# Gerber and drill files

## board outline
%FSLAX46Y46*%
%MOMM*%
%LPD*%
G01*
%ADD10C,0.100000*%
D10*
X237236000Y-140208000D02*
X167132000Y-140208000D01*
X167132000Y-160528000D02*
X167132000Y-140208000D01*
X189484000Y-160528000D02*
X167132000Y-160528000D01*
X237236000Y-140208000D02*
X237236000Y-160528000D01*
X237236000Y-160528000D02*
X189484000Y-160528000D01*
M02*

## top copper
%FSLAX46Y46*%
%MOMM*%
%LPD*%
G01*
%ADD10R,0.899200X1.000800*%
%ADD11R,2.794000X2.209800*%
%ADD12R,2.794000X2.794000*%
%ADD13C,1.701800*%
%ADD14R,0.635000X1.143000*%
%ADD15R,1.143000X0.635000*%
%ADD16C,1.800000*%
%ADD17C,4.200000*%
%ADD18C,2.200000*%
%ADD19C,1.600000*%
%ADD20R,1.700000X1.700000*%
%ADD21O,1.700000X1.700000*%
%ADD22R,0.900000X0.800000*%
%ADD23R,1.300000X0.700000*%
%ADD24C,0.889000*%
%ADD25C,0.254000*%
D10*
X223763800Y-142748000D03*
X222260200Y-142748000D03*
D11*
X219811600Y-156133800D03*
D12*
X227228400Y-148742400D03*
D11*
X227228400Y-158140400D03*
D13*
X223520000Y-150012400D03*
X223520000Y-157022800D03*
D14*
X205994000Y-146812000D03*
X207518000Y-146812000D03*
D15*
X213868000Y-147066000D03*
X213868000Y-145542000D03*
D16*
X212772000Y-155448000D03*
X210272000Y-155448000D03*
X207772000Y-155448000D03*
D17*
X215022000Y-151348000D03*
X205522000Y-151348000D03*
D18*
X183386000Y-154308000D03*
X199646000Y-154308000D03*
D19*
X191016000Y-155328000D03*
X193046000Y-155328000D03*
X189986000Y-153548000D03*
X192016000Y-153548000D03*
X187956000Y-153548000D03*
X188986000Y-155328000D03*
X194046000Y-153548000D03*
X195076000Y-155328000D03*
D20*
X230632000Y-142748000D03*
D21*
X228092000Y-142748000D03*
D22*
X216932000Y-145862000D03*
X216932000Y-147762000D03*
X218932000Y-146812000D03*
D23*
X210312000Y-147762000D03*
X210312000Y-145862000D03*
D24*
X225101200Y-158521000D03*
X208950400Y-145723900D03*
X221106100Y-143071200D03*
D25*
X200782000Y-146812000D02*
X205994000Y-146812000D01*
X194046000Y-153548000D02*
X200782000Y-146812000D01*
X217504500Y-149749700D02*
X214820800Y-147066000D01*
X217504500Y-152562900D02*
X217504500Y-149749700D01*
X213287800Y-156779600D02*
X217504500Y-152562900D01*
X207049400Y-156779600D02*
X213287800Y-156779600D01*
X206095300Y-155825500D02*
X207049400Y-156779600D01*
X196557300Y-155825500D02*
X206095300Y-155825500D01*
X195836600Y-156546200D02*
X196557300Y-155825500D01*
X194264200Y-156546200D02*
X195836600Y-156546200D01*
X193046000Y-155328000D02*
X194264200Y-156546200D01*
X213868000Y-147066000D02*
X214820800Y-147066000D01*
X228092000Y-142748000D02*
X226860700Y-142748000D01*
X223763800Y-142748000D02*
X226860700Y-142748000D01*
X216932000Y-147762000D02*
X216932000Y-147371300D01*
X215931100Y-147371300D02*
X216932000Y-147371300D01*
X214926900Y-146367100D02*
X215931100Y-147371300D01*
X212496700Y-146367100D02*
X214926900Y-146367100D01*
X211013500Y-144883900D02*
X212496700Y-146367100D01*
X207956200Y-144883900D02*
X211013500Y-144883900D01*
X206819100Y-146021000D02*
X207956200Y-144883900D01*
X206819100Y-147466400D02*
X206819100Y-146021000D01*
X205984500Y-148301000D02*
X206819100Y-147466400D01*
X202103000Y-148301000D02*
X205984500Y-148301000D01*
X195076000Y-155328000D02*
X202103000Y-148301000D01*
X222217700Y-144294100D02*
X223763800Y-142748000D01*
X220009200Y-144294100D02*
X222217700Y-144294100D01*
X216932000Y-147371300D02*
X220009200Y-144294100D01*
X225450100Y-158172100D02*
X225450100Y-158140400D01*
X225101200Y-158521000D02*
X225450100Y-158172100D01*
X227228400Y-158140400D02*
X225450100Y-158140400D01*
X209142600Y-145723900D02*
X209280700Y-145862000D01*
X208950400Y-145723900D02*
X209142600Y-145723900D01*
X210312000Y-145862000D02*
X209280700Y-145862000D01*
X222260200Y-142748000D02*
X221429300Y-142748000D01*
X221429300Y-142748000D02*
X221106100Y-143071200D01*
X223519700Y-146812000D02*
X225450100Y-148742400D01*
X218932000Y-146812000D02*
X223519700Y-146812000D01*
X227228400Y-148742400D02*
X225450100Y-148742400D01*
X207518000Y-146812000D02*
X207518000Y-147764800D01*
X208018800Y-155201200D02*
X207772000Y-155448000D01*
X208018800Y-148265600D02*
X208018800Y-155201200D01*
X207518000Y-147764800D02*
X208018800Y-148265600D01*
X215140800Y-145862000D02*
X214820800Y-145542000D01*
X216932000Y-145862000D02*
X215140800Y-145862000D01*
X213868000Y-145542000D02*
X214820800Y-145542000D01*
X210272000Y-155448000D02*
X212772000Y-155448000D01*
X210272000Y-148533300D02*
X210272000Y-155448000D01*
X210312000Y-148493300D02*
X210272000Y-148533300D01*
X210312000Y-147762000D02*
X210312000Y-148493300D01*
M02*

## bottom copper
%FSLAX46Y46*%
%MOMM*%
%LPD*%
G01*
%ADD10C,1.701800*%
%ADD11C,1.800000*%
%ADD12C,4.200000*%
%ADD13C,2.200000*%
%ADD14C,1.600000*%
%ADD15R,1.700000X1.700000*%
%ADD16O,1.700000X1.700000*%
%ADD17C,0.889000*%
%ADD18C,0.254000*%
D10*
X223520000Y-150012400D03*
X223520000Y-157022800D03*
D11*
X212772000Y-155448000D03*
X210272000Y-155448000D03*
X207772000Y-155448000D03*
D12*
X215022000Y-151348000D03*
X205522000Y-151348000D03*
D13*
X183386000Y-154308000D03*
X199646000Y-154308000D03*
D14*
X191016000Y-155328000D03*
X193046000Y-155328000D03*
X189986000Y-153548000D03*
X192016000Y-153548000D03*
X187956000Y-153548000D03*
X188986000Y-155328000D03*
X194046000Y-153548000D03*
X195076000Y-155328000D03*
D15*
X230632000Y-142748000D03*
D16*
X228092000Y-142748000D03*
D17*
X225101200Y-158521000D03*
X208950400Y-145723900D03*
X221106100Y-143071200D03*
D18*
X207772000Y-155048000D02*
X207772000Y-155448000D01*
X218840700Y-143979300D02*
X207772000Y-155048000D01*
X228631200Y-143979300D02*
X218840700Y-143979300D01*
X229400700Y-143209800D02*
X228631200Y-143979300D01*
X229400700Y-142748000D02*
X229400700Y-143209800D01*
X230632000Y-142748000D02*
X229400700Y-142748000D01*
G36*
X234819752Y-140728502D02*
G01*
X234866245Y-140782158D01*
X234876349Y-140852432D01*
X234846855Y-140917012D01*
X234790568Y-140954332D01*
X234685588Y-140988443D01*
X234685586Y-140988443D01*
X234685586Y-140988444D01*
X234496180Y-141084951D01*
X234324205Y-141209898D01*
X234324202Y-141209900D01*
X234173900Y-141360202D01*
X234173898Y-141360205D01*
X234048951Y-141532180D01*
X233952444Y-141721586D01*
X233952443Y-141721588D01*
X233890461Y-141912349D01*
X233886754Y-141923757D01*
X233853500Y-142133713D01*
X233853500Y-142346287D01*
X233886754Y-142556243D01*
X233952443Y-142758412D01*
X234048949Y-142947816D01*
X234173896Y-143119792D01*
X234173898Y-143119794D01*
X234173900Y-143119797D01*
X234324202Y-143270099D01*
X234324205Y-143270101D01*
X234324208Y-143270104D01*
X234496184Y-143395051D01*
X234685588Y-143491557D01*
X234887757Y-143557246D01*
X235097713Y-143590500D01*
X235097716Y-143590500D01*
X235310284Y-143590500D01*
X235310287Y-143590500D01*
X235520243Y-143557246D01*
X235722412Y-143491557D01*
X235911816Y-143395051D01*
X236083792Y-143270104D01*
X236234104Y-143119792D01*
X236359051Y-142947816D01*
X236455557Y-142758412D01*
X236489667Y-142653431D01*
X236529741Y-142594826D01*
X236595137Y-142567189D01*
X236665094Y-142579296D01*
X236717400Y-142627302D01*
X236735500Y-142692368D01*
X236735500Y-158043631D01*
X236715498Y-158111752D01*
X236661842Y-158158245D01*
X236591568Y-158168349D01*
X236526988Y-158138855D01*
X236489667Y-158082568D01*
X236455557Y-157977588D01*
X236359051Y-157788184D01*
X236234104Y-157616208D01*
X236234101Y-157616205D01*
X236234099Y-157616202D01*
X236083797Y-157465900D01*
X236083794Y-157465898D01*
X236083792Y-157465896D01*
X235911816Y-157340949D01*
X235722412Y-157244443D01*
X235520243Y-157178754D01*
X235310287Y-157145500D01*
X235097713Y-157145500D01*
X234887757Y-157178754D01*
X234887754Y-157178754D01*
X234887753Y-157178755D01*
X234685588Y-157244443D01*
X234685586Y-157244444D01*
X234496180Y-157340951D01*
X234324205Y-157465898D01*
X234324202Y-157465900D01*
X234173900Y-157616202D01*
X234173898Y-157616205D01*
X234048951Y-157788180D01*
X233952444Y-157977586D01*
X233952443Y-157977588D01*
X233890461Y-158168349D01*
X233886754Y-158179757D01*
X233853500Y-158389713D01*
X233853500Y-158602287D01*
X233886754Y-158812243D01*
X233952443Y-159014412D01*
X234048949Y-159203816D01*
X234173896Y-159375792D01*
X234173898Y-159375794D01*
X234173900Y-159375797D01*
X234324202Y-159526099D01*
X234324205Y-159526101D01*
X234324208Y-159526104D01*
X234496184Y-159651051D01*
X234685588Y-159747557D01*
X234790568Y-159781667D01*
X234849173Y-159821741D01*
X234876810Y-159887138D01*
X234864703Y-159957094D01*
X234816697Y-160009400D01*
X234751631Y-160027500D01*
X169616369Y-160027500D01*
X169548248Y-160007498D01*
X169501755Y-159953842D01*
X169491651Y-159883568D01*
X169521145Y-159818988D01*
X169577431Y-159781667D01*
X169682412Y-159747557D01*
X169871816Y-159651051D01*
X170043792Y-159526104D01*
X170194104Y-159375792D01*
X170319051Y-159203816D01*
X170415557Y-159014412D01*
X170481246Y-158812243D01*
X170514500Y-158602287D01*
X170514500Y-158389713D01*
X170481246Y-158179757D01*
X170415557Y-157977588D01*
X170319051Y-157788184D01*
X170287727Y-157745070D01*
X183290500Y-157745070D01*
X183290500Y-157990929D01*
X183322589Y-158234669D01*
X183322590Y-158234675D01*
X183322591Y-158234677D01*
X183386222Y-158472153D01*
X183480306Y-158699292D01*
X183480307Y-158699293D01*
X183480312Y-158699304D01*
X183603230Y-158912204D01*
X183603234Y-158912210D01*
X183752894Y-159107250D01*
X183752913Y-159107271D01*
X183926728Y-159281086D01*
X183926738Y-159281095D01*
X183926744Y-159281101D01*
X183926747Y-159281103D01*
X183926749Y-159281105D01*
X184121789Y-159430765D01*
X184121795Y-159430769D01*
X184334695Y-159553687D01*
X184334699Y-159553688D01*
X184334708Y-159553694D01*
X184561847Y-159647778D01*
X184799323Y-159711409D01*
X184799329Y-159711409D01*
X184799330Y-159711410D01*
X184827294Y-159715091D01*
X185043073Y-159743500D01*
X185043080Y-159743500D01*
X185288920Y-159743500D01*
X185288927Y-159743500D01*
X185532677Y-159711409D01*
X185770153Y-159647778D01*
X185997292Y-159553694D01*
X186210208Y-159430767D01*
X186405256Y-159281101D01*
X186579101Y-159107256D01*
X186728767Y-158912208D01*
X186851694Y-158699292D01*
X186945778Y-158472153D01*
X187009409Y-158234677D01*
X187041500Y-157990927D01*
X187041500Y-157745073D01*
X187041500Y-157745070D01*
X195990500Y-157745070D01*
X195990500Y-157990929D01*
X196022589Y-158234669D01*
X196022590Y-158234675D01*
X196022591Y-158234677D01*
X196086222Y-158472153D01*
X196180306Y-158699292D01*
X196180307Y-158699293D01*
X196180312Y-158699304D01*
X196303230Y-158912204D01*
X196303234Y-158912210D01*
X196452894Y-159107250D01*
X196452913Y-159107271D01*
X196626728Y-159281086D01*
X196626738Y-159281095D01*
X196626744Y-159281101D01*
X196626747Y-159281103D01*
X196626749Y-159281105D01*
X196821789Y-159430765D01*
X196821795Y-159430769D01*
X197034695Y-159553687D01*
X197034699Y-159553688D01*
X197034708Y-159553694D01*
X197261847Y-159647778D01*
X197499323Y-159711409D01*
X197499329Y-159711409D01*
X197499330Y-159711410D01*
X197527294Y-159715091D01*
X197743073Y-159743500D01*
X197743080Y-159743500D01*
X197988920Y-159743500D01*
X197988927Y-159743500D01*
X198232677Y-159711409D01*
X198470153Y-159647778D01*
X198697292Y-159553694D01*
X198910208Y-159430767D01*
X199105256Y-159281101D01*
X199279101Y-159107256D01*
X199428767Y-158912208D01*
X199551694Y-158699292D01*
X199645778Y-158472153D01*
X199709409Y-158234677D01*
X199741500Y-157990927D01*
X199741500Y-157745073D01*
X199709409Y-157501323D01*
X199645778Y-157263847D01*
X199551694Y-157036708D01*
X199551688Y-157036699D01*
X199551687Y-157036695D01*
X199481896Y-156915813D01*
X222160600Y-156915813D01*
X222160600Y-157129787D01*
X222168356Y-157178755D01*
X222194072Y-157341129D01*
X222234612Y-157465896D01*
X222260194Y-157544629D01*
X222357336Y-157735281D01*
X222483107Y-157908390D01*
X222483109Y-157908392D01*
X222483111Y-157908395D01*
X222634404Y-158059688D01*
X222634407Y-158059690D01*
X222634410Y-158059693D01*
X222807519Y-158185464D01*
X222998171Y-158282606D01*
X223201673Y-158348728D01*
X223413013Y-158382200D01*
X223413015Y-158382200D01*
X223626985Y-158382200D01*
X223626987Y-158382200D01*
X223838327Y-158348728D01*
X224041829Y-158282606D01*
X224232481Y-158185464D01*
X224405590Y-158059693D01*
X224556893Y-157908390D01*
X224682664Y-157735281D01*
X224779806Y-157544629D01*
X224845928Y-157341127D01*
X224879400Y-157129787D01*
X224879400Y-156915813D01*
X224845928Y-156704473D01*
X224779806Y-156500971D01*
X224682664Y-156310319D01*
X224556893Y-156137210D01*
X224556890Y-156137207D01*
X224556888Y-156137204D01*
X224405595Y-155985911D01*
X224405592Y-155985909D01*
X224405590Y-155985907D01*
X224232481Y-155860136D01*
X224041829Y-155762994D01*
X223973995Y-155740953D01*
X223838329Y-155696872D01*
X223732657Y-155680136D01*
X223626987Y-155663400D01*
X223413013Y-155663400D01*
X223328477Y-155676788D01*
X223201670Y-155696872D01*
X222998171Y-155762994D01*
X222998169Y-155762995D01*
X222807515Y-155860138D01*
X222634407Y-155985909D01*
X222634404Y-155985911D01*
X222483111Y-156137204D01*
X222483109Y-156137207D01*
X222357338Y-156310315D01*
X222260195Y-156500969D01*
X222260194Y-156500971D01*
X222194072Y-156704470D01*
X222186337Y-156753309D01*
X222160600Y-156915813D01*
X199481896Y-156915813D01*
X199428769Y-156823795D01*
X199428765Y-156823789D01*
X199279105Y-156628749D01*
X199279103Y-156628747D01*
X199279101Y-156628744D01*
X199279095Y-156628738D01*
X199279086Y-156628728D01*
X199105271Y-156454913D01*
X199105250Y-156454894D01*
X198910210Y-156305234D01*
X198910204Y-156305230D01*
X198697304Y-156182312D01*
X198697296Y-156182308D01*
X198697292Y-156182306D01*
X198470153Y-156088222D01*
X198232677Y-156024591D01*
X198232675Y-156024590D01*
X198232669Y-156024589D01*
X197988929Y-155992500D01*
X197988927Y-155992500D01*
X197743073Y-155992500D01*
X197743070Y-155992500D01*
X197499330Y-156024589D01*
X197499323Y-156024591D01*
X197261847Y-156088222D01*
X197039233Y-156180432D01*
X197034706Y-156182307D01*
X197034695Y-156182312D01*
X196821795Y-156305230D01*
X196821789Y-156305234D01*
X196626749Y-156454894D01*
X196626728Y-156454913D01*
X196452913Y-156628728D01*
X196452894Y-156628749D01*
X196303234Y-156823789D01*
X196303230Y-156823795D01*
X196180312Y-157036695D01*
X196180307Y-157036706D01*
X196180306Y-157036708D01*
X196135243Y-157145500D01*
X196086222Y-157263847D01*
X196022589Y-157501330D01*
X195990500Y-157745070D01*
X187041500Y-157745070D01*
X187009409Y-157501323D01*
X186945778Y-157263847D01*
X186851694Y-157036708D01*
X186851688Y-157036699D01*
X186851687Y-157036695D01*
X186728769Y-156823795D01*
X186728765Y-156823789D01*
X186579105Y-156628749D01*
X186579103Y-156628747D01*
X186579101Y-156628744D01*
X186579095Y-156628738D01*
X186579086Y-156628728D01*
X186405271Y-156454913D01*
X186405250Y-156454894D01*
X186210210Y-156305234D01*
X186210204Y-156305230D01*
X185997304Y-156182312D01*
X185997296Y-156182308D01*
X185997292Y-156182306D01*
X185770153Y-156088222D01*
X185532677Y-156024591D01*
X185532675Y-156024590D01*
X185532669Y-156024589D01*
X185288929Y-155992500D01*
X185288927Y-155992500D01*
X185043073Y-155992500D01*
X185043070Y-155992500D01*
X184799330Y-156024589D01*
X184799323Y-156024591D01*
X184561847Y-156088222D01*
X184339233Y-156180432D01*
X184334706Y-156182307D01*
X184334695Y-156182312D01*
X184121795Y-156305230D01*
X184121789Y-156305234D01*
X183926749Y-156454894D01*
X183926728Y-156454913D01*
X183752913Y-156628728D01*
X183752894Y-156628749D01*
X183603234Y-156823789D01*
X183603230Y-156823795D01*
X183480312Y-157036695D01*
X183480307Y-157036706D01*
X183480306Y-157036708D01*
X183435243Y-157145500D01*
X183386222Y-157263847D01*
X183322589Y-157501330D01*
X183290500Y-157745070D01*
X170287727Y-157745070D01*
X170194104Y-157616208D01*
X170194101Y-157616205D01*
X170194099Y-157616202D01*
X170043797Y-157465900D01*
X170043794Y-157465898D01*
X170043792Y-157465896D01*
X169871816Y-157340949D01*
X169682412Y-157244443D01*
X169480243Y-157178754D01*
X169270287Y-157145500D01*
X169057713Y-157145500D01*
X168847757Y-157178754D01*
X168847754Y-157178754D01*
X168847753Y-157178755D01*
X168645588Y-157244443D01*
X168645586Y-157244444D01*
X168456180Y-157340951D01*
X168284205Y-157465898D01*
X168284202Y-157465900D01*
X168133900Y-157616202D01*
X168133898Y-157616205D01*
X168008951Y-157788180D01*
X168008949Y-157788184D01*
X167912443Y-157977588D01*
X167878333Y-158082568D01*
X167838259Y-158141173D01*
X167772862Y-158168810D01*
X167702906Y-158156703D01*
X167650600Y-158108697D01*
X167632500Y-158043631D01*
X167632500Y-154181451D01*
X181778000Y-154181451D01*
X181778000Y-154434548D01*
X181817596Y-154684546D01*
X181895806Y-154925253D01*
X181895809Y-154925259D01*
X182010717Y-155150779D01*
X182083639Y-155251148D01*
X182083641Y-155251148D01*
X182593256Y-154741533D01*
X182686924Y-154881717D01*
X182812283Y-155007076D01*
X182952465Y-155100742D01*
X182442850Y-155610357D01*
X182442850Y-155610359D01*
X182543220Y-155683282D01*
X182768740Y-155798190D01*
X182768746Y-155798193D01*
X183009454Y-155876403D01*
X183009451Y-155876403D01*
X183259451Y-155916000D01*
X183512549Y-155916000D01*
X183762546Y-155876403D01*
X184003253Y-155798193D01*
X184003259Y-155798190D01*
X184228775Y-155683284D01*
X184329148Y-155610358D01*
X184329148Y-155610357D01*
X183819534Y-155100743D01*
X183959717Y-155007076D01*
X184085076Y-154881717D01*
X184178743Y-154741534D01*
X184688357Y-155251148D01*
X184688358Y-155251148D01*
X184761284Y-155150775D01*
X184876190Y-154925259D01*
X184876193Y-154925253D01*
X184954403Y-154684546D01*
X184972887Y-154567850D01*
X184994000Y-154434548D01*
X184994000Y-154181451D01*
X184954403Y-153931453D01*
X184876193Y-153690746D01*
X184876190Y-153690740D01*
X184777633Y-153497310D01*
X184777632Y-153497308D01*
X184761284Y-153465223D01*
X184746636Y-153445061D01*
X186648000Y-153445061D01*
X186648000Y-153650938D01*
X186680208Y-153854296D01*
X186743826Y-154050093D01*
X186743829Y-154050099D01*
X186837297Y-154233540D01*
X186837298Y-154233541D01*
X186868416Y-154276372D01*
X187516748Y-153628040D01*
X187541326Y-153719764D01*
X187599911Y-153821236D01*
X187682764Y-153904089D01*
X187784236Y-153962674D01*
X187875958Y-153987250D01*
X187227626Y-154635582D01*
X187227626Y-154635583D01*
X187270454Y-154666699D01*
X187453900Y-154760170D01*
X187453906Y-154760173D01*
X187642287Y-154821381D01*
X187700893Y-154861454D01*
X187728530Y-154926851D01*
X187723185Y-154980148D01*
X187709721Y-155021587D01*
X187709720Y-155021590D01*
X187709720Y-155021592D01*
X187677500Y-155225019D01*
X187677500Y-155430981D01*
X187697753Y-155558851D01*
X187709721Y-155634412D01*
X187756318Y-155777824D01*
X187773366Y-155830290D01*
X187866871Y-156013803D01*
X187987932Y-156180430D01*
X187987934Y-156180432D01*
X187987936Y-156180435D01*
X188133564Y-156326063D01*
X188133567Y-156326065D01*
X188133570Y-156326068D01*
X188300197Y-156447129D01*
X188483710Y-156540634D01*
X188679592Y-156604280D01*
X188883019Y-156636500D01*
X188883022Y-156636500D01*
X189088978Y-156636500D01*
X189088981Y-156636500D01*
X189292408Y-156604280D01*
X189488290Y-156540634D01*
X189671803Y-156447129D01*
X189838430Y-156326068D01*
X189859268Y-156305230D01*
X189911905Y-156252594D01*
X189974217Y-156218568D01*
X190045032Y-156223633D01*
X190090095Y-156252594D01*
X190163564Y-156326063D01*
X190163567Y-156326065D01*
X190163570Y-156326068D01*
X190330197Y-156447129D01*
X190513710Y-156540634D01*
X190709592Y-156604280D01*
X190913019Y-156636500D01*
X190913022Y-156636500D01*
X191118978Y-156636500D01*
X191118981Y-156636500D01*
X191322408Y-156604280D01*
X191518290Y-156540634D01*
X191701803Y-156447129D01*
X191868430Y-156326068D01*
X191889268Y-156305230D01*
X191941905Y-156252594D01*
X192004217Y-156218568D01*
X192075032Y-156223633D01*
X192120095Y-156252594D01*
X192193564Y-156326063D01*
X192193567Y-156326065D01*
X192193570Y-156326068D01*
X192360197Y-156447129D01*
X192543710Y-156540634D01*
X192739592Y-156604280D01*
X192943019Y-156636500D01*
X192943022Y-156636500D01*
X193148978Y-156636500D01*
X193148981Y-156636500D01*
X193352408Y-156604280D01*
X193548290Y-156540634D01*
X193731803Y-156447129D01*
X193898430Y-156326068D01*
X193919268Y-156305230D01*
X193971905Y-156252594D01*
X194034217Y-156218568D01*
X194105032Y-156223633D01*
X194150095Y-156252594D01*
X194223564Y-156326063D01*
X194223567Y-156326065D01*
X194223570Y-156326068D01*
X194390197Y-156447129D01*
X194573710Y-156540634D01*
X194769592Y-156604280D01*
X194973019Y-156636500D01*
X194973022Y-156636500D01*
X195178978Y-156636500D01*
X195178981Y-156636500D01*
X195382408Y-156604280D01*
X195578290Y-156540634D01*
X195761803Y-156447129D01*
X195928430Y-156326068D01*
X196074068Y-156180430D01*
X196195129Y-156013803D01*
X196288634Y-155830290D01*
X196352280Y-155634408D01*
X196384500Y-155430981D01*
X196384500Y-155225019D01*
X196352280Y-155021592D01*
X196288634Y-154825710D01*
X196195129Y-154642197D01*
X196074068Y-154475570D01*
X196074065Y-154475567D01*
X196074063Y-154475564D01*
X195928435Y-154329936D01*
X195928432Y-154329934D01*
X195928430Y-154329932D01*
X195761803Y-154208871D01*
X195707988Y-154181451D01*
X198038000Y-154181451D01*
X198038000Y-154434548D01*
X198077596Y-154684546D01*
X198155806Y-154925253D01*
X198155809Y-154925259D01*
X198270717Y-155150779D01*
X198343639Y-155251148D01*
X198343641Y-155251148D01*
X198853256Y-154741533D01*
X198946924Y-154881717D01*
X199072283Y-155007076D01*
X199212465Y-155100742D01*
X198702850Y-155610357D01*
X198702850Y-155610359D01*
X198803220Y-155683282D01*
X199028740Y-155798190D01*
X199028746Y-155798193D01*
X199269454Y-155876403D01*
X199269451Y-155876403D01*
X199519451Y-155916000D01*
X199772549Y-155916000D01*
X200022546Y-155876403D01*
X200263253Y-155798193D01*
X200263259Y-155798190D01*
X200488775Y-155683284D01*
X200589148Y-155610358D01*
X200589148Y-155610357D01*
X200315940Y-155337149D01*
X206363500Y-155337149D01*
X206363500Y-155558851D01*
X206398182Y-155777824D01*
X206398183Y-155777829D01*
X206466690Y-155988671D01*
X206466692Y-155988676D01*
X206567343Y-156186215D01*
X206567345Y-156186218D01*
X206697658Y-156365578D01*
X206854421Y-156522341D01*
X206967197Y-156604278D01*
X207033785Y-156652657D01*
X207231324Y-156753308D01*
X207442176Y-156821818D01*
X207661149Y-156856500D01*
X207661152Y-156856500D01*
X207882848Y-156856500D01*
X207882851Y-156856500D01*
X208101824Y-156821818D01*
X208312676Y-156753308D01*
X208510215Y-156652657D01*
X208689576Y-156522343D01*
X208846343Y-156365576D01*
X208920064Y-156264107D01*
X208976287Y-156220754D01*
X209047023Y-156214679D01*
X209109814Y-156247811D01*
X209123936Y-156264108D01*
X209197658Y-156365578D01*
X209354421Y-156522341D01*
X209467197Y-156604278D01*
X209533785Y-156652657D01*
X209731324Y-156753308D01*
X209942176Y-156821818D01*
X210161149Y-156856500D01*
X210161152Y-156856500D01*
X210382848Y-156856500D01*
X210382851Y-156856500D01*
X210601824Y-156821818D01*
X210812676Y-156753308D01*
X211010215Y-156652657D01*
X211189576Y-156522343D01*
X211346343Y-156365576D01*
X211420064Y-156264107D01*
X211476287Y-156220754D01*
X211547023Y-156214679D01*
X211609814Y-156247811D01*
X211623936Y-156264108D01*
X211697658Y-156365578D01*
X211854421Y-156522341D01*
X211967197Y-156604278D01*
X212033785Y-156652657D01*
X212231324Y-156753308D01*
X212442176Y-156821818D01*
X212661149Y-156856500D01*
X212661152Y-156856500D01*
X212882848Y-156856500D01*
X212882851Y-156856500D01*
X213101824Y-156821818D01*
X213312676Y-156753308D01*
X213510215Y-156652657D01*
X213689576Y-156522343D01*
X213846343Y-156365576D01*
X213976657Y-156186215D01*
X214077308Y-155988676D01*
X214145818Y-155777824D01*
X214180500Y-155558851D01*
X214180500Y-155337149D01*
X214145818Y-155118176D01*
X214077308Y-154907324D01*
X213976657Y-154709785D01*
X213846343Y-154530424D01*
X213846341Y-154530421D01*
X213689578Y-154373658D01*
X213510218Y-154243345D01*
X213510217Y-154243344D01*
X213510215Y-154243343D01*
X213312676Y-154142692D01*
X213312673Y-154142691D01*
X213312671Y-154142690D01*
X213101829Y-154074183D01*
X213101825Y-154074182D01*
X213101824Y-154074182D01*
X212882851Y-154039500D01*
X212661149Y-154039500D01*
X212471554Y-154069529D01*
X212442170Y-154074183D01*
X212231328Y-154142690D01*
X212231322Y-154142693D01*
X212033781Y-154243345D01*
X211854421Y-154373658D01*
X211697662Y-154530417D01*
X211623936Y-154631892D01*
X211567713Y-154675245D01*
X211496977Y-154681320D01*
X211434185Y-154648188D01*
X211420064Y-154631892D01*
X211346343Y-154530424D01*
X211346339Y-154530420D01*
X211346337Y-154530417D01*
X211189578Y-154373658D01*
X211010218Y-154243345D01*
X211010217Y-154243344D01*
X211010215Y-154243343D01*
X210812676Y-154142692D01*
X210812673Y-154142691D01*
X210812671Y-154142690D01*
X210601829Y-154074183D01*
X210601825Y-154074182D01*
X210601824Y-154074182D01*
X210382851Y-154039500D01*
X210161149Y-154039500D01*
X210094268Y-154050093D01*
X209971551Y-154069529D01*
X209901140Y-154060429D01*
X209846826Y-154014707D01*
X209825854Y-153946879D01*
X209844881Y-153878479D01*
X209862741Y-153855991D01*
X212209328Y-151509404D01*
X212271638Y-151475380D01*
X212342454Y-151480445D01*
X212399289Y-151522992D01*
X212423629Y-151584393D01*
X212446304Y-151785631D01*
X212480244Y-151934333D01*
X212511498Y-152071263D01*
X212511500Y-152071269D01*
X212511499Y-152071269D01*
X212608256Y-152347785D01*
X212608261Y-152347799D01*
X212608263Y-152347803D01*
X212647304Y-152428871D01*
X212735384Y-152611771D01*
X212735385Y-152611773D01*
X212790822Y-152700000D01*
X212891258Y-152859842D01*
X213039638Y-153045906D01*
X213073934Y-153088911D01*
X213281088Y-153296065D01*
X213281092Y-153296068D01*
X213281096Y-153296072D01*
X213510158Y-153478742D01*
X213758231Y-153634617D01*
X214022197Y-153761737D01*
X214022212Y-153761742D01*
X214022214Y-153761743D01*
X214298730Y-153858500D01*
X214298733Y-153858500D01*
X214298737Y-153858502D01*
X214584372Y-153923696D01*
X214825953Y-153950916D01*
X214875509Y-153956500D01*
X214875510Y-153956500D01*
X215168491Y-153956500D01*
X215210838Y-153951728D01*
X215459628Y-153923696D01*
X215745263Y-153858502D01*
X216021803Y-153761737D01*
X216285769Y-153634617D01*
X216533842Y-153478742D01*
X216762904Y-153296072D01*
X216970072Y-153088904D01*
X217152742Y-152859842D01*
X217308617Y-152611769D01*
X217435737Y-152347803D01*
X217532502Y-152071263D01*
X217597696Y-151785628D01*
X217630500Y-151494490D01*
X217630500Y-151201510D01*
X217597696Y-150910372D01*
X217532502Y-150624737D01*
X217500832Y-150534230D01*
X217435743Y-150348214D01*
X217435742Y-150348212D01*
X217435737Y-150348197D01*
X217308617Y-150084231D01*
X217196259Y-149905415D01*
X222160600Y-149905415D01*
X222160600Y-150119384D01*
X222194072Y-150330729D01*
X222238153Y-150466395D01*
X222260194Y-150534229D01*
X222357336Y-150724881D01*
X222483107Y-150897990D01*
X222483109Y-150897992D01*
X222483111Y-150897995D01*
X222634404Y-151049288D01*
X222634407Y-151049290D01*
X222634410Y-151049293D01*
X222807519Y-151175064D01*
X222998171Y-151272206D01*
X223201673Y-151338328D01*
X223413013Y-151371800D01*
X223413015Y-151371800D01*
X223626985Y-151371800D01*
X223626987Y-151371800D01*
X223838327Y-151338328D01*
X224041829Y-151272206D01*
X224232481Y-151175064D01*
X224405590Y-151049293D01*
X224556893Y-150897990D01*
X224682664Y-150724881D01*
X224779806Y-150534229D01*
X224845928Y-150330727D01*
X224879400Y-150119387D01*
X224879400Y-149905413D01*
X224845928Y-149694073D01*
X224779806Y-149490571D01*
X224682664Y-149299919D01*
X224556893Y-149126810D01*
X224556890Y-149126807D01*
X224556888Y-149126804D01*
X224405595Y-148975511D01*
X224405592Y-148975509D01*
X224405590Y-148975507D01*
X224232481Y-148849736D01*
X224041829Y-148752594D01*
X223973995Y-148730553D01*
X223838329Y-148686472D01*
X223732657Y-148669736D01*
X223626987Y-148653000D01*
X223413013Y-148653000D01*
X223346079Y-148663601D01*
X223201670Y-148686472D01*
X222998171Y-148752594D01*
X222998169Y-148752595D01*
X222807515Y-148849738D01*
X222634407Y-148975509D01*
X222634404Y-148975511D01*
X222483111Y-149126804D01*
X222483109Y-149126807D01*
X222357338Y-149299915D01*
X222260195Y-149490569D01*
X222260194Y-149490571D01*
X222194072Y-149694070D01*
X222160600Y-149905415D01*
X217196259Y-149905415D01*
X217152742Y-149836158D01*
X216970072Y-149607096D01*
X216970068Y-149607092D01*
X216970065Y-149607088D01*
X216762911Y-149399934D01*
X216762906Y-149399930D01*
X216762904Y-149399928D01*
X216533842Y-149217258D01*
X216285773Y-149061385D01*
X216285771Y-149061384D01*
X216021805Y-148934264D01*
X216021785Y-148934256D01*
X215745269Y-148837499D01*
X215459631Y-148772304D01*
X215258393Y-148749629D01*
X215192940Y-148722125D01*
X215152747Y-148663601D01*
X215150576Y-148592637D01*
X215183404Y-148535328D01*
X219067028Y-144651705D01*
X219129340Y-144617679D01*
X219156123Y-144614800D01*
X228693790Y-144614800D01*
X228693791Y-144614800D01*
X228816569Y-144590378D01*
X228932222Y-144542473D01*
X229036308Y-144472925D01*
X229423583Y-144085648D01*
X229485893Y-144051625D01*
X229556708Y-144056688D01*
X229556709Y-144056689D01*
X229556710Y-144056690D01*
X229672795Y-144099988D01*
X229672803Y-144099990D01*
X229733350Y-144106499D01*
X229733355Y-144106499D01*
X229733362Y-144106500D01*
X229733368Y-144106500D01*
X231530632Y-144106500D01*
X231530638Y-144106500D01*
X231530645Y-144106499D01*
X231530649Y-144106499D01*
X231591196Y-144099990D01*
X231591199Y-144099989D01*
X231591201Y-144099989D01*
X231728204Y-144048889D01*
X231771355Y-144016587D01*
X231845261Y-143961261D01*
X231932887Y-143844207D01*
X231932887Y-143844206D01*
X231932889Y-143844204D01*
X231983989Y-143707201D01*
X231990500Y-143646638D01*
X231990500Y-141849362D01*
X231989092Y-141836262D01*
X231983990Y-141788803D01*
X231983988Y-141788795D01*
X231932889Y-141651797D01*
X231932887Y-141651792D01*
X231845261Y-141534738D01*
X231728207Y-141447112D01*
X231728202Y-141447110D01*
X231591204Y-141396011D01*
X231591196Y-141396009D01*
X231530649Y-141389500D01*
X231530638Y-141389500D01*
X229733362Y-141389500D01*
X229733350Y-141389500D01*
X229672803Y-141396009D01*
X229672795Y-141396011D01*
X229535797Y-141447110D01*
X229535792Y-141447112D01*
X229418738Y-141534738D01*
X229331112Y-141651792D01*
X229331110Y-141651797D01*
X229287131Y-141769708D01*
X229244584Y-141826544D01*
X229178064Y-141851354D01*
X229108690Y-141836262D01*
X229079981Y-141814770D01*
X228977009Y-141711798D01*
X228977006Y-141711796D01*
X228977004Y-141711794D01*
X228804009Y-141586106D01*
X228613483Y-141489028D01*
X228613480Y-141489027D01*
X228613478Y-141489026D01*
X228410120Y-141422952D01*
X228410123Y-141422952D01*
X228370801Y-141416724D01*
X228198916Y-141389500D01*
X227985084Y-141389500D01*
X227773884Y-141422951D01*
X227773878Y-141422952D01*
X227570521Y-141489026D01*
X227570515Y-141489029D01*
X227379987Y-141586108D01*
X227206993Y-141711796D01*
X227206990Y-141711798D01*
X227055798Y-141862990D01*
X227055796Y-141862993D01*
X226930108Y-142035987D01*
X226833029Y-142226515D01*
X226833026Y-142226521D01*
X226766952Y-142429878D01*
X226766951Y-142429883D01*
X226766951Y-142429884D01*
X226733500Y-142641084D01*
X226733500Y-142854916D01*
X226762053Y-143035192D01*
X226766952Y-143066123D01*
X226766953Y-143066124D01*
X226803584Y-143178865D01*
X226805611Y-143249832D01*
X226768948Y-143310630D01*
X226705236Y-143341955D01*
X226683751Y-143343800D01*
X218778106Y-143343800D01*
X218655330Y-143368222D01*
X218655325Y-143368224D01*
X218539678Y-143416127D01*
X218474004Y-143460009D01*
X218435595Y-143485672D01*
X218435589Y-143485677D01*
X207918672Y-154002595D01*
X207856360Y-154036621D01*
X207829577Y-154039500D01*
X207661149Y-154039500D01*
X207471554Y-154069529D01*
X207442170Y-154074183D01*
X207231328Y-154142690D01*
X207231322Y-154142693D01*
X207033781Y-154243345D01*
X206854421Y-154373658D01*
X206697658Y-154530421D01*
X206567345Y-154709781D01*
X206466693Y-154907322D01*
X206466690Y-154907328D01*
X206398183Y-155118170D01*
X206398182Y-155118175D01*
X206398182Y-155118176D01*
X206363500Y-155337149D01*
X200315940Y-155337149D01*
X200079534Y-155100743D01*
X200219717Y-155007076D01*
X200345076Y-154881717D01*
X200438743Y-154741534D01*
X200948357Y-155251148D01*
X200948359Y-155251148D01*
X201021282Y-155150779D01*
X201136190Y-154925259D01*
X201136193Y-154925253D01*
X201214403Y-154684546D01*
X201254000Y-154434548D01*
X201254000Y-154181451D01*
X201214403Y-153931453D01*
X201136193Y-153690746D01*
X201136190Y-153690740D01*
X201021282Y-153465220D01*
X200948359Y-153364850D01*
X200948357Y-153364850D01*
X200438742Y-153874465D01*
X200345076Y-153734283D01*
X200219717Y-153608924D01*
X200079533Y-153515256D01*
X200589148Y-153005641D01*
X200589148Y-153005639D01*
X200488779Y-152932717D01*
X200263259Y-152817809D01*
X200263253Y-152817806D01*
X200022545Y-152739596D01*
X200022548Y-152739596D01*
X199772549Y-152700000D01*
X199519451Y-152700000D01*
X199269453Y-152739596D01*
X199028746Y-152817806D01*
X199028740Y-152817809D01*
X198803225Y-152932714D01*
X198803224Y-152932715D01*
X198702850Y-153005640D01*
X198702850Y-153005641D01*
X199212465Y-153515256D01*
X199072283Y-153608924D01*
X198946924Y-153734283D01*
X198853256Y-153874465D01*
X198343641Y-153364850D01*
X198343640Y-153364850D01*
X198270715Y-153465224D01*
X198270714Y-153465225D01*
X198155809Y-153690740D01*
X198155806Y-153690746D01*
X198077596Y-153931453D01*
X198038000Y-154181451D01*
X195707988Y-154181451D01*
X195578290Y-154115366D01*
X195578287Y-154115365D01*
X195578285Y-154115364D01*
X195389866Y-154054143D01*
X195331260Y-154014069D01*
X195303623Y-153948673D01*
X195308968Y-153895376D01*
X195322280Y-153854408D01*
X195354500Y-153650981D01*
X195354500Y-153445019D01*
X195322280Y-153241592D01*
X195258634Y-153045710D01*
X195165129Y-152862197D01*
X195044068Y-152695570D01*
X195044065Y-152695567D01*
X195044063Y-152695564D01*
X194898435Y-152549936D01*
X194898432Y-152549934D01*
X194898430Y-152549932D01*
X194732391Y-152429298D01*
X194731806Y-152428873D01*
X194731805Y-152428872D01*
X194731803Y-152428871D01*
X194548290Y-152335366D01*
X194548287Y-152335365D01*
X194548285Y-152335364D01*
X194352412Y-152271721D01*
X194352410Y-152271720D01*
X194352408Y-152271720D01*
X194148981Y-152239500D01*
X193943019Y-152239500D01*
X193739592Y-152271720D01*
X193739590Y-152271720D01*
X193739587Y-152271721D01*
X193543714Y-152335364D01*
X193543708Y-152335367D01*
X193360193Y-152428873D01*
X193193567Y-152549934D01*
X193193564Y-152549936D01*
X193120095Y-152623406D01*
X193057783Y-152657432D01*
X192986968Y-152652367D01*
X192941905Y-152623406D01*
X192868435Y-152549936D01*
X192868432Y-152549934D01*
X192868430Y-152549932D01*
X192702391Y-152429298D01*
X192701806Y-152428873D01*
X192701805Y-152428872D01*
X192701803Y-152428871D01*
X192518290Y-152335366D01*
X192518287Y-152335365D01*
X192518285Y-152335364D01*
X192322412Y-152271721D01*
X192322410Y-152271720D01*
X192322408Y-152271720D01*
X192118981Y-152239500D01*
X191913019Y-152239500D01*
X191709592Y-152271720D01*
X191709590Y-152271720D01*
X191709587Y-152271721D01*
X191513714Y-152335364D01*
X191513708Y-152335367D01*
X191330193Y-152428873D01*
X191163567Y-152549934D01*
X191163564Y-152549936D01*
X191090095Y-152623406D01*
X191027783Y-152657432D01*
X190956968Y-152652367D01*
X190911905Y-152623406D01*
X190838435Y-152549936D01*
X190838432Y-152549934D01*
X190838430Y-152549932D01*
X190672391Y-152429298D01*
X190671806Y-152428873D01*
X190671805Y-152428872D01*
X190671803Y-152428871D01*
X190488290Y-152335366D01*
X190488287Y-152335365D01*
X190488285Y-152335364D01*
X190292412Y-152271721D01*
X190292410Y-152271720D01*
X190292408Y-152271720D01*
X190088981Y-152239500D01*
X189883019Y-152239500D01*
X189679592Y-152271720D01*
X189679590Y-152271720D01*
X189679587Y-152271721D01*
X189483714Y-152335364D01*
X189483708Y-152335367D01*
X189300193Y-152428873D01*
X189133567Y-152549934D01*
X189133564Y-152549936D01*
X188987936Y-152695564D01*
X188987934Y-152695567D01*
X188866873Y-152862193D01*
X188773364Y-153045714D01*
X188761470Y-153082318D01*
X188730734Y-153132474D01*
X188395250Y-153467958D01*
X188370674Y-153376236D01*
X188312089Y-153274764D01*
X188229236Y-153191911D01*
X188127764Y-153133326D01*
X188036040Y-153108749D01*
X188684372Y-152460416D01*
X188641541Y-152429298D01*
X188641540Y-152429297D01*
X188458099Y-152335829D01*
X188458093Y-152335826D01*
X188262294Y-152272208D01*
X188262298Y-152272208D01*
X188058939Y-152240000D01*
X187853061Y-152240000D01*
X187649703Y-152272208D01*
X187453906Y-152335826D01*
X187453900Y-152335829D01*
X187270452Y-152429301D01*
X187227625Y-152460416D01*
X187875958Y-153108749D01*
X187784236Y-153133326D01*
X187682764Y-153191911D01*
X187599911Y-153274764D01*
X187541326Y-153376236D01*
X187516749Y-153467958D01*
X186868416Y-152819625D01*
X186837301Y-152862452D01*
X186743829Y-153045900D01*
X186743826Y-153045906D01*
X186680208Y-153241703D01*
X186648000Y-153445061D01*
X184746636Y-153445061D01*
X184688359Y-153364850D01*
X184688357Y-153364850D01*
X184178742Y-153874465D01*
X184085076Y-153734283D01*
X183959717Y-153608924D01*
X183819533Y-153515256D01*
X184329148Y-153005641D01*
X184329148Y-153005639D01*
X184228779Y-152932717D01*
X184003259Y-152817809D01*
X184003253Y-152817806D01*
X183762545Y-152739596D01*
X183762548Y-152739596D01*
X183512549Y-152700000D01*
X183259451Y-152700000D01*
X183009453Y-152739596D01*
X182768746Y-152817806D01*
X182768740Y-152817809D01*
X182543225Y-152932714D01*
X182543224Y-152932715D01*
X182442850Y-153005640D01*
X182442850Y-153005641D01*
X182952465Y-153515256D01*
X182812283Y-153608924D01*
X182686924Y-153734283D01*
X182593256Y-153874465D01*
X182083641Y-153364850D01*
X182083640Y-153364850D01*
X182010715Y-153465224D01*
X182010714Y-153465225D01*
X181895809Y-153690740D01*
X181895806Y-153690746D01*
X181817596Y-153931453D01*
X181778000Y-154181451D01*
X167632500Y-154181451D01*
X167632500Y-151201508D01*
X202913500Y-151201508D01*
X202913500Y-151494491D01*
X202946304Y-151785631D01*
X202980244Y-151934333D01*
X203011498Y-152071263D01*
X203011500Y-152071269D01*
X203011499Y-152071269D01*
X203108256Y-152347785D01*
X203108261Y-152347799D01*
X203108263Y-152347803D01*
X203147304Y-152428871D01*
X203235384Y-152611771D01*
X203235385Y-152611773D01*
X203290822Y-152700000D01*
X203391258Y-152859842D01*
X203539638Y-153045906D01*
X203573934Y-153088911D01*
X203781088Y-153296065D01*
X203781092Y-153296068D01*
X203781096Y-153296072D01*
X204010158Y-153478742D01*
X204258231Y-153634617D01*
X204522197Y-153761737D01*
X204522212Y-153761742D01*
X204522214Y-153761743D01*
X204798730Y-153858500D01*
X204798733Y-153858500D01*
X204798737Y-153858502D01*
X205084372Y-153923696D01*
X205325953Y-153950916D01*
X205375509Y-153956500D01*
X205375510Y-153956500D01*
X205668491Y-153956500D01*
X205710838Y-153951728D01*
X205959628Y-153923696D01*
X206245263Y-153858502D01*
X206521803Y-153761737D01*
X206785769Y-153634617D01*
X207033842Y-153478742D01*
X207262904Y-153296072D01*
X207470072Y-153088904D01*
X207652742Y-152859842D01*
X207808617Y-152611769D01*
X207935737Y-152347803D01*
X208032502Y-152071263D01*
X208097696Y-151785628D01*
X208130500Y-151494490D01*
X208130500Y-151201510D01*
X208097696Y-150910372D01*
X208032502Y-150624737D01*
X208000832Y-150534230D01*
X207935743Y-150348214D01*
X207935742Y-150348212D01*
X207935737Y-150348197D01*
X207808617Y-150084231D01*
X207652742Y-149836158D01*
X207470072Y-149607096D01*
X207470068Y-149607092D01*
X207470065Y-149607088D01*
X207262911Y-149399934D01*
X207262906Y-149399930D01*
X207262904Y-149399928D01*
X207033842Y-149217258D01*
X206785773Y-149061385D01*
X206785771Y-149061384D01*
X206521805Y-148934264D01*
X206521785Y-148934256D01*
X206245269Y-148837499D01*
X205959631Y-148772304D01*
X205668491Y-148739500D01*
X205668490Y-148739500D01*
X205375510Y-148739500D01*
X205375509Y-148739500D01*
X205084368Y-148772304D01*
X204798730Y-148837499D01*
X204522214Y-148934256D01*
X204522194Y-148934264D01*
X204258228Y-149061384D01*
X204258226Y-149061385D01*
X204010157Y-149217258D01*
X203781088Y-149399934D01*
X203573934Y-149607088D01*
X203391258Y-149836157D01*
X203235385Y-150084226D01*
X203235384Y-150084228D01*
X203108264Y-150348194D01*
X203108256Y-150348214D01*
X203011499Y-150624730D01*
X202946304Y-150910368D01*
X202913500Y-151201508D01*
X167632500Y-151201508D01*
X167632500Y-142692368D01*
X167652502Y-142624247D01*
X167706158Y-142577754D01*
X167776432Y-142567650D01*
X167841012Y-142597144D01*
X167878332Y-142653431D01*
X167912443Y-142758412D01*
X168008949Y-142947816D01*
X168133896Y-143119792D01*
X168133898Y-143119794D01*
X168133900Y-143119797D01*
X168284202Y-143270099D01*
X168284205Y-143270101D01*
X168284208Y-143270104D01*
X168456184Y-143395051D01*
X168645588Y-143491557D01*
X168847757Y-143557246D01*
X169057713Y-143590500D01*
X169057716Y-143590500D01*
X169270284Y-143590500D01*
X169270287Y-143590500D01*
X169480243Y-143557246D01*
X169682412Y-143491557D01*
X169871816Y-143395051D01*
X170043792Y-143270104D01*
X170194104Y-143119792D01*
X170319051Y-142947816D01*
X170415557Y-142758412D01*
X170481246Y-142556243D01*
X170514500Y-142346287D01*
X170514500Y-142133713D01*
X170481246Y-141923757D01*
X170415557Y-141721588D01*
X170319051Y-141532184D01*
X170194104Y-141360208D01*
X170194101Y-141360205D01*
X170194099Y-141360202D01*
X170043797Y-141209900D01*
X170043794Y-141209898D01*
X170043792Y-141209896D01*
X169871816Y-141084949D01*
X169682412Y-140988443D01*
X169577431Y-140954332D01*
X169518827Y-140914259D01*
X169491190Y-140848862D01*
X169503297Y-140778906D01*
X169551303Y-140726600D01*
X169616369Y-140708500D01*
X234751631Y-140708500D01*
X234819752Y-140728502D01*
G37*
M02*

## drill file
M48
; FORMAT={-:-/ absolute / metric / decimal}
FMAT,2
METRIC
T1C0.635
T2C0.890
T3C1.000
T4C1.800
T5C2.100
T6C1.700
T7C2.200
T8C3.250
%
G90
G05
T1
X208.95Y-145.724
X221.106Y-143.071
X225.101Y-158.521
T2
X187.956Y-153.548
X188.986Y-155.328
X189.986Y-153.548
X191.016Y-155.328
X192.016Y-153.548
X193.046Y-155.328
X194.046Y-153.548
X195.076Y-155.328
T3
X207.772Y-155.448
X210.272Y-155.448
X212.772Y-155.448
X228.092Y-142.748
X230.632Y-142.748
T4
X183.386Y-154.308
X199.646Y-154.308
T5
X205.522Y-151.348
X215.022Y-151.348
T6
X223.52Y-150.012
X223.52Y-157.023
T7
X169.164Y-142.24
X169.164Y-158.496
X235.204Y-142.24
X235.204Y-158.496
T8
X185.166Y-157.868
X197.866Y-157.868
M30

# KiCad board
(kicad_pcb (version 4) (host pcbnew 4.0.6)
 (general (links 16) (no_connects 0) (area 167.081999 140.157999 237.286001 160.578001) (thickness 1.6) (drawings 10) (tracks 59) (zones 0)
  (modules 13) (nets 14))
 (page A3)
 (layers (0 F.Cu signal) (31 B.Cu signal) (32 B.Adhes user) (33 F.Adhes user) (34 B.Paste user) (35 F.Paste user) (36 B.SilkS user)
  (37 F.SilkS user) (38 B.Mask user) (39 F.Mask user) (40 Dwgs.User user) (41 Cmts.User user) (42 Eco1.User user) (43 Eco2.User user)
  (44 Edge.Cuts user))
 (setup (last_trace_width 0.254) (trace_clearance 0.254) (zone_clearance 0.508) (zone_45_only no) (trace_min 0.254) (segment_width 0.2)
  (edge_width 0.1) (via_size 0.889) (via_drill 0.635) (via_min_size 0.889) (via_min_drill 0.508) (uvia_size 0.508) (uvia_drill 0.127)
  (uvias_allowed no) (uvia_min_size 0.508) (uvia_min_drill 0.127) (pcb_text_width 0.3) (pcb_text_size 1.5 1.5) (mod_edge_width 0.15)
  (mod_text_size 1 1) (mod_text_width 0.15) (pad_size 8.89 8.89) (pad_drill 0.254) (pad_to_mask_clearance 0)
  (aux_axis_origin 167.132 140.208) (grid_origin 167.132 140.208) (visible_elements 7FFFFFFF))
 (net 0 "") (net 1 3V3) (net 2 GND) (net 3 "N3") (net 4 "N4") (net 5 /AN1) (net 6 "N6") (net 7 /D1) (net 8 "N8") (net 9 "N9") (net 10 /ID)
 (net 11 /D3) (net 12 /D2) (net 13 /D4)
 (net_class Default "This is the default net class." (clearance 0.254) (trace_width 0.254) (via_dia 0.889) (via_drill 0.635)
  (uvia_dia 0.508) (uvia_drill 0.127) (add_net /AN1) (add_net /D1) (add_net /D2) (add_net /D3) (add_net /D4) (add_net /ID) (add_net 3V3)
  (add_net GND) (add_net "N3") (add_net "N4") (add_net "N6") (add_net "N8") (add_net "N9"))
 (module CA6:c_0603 (layer F.Cu) (at 223.012 142.748)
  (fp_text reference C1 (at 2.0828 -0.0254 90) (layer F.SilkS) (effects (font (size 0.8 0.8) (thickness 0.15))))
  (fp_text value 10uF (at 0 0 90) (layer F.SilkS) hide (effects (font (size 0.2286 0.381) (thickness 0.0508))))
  (pad 1 smd rect (at 0.7518 0) (size 0.8992 1.0008) (layers F.Cu F.Paste F.Mask) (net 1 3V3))
  (pad 2 smd rect (at -0.7518 0) (size 0.8992 1.0008) (layers F.Cu F.Paste F.Mask) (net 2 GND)))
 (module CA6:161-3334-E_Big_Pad (layer F.Cu) (at 223.52 160.528 90)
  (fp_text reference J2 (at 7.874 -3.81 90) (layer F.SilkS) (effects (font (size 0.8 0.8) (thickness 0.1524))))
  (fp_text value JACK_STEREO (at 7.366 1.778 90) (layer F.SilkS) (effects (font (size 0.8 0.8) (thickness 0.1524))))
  (pad 1 smd rect (at 4.3942 -3.7084 90) (size 2.2098 2.794) (layers F.Cu F.Paste F.Mask) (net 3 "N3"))
  (pad 2 smd rect (at 11.7856 3.7084 90) (size 2.794 2.794) (layers F.Cu F.Paste F.Mask) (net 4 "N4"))
  (pad 3 smd rect (at 2.3876 3.7084 90) (size 2.2098 2.794) (layers F.Cu F.Paste F.Mask) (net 2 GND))
  (pad "" np_thru_hole circle (at 10.5156 0) (size 1.7018 1.7018) (drill 1.7) (layers *.Cu *.Mask F.SilkS))
  (pad "" np_thru_hole circle (at 3.5052 0) (size 1.7018 1.7018) (drill 1.7) (layers *.Cu *.Mask F.SilkS)))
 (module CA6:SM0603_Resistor (layer F.Cu) (at 206.756 146.812)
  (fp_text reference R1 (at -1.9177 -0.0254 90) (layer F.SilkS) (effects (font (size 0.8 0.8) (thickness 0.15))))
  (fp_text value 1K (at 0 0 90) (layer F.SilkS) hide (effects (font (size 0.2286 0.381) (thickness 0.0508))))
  (pad 1 smd rect (at -0.762 0) (size 0.635 1.143) (layers F.Cu F.Paste F.Mask) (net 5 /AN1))
  (pad 2 smd rect (at 0.762 0) (size 0.635 1.143) (layers F.Cu F.Paste F.Mask) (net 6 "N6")))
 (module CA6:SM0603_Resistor (layer F.Cu) (at 213.868 146.304 90)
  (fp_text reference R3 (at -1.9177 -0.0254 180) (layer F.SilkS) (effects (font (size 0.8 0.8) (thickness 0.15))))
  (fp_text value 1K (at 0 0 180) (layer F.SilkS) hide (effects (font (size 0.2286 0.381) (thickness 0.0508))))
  (pad 1 smd rect (at -0.762 0 90) (size 0.635 1.143) (layers F.Cu F.Paste F.Mask) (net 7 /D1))
  (pad 2 smd rect (at 0.762 0 90) (size 0.635 1.143) (layers F.Cu F.Paste F.Mask) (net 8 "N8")))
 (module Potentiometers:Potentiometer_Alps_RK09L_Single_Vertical (layer F.Cu) (at 207.772 155.448 270)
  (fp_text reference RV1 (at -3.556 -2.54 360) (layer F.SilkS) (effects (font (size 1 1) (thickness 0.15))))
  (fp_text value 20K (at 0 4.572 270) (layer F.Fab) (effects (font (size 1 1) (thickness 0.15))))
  (pad 3 thru_hole circle (at 0 -5 270) (size 1.8 1.8) (drill 1) (layers *.Cu *.Mask) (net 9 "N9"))
  (pad 2 thru_hole circle (at 0 -2.5 270) (size 1.8 1.8) (drill 1) (layers *.Cu *.Mask) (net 9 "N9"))
  (pad 1 thru_hole circle (at 0 0 270) (size 1.8 1.8) (drill 1) (layers *.Cu *.Mask) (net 6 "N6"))
  (pad 0 thru_hole circle (at -4.1 -7.25 270) (size 4.2 4.2) (drill 2.1) (layers *.Cu *.Mask))
  (pad 0 thru_hole circle (at -4.1 2.25 270) (size 4.2 4.2) (drill 2.1) (layers *.Cu *.Mask)))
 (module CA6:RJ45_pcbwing (layer F.Cu) (at 191.516 155.448)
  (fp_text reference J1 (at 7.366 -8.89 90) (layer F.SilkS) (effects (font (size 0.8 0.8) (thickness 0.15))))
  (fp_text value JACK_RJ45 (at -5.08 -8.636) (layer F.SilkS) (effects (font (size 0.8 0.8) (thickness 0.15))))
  (pad 8 thru_hole circle (at -8.13 -1.14) (size 2.2 2.2) (drill 1.8) (layers *.Cu *.Mask F.SilkS) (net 2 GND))
  (pad 8 thru_hole circle (at 8.13 -1.14) (size 2.2 2.2) (drill 1.8) (layers *.Cu *.Mask F.SilkS) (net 2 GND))
  (pad "" np_thru_hole circle (at -6.35 2.42) (size 3.25 3.25) (drill 3.25) (layers *.Cu *.Mask F.SilkS))
  (pad "" np_thru_hole circle (at 6.35 2.42) (size 3.25 3.25) (drill 3.25) (layers *.Cu *.Mask F.SilkS))
  (pad 5 thru_hole circle (at -0.5 -0.12) (size 1.6 1.6) (drill 0.89) (layers *.Cu *.Mask F.SilkS) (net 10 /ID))
  (pad 3 thru_hole circle (at 1.53 -0.12) (size 1.6 1.6) (drill 0.89) (layers *.Cu *.Mask F.SilkS) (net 7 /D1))
  (pad 6 thru_hole circle (at -1.53 -1.9) (size 1.6 1.6) (drill 0.89) (layers *.Cu *.Mask F.SilkS) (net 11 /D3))
  (pad 4 thru_hole circle (at 0.5 -1.9) (size 1.6 1.6) (drill 0.89) (layers *.Cu *.Mask F.SilkS) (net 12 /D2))
  (pad 8 thru_hole circle (at -3.56 -1.9) (size 1.6 1.6) (drill 0.89) (layers *.Cu *.Mask F.SilkS) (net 2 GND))
  (pad 7 thru_hole circle (at -2.53 -0.12) (size 1.6 1.6) (drill 0.89) (layers *.Cu *.Mask F.SilkS) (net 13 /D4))
  (pad 2 thru_hole circle (at 2.53 -1.9) (size 1.6 1.6) (drill 0.89) (layers *.Cu *.Mask F.SilkS) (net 5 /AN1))
  (pad 1 thru_hole circle (at 3.56 -0.12) (size 1.6 1.6) (drill 0.89) (layers *.Cu *.Mask F.SilkS) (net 1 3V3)))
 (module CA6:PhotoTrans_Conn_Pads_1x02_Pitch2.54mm (layer F.Cu) (at 230.632 142.748 270)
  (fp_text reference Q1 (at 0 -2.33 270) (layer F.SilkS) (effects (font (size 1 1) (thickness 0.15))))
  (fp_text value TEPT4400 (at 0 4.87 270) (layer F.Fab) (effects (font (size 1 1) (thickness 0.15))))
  (pad 1 thru_hole rect (at 0 0 270) (size 1.7 1.7) (drill 1) (layers *.Cu *.Mask) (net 6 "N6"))
  (pad 3 thru_hole oval (at 0 2.54 270) (size 1.7 1.7) (drill 1) (layers *.Cu *.Mask) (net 1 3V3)))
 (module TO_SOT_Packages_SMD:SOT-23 (layer F.Cu) (at 217.932 146.812)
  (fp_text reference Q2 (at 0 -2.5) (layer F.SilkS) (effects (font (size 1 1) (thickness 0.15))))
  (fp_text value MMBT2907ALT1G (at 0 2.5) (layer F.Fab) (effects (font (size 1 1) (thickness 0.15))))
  (pad 1 smd rect (at -1 -0.95) (size 0.9 0.8) (layers F.Cu F.Paste F.Mask) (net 8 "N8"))
  (pad 2 smd rect (at -1 0.95) (size 0.9 0.8) (layers F.Cu F.Paste F.Mask) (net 1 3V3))
  (pad 3 smd rect (at 1 0) (size 0.9 0.8) (layers F.Cu F.Paste F.Mask) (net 4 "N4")))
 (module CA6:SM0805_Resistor (layer F.Cu) (at 210.312 146.812 90)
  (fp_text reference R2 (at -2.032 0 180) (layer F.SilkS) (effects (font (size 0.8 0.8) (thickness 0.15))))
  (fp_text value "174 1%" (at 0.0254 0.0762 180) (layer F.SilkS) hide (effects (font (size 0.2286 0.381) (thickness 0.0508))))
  (pad 1 smd rect (at -0.95 0 90) (size 0.7 1.3) (layers F.Cu F.Paste F.Mask) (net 9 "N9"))
  (pad 2 smd rect (at 0.95 0 90) (size 0.7 1.3) (layers F.Cu F.Paste F.Mask) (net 2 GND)))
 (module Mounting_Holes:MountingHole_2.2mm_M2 (layer F.Cu) (at 169.164 142.24)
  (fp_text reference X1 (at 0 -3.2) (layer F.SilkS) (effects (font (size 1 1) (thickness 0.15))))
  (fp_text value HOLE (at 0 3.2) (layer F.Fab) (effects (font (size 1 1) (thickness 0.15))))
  (pad 1 np_thru_hole circle (at 0 0) (size 2.2 2.2) (drill 2.2) (layers *.Cu *.Mask)))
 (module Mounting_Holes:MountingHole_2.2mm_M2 (layer F.Cu) (at 169.164 158.496)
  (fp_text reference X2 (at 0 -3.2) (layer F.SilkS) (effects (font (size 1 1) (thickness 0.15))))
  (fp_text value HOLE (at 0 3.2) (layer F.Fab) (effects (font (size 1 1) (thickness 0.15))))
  (pad 1 np_thru_hole circle (at 0 0) (size 2.2 2.2) (drill 2.2) (layers *.Cu *.Mask)))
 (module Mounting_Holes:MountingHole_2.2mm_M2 (layer F.Cu) (at 235.204 142.24)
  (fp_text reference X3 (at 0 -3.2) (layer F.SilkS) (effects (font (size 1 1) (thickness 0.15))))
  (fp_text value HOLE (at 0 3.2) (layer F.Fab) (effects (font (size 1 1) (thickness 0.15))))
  (pad 1 np_thru_hole circle (at 0 0) (size 2.2 2.2) (drill 2.2) (layers *.Cu *.Mask)))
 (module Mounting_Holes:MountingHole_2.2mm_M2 (layer F.Cu) (at 235.204 158.496)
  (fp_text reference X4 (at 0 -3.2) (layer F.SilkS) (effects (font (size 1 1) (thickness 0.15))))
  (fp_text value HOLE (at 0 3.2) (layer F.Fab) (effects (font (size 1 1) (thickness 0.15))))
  (pad 1 np_thru_hole circle (at 0 0) (size 2.2 2.2) (drill 2.2) (layers *.Cu *.Mask)))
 (gr_line (start 237.236 140.208) (end 167.132 140.208) (angle 90) (layer Edge.Cuts) (width 0.1))
 (gr_line (start 167.132 160.528) (end 167.132 140.208) (angle 90) (layer Edge.Cuts) (width 0.1))
 (gr_line (start 189.484 160.528) (end 167.132 160.528) (angle 90) (layer Edge.Cuts) (width 0.1))
 (gr_line (start 237.236 140.208) (end 237.236 160.528) (angle 90) (layer Edge.Cuts) (width 0.1))
 (gr_line (start 237.236 160.528) (end 189.484 160.528) (angle 90) (layer Edge.Cuts) (width 0.1))
 (segment (start 200.782 146.812) (end 205.994 146.812) (width 0.254) (layer F.Cu) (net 5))
 (segment (start 194.046 153.548) (end 200.782 146.812) (width 0.254) (layer F.Cu) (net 5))
 (segment (start 217.5045 149.7497) (end 214.8208 147.066) (width 0.254) (layer F.Cu) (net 7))
 (segment (start 217.5045 152.5629) (end 217.5045 149.7497) (width 0.254) (layer F.Cu) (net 7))
 (segment (start 213.2878 156.7796) (end 217.5045 152.5629) (width 0.254) (layer F.Cu) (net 7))
 (segment (start 207.0494 156.7796) (end 213.2878 156.7796) (width 0.254) (layer F.Cu) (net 7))
 (segment (start 206.0953 155.8255) (end 207.0494 156.7796) (width 0.254) (layer F.Cu) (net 7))
 (segment (start 196.5573 155.8255) (end 206.0953 155.8255) (width 0.254) (layer F.Cu) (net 7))
 (segment (start 195.8366 156.5462) (end 196.5573 155.8255) (width 0.254) (layer F.Cu) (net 7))
 (segment (start 194.2642 156.5462) (end 195.8366 156.5462) (width 0.254) (layer F.Cu) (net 7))
 (segment (start 193.046 155.328) (end 194.2642 156.5462) (width 0.254) (layer F.Cu) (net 7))
 (segment (start 213.868 147.066) (end 214.8208 147.066) (width 0.254) (layer F.Cu) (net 7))
 (segment (start 228.092 142.748) (end 226.8607 142.748) (width 0.254) (layer F.Cu) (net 1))
 (segment (start 223.7638 142.748) (end 226.8607 142.748) (width 0.254) (layer F.Cu) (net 1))
 (segment (start 216.932 147.762) (end 216.932 147.3713) (width 0.254) (layer F.Cu) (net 1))
 (segment (start 215.9311 147.3713) (end 216.932 147.3713) (width 0.254) (layer F.Cu) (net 1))
 (segment (start 214.9269 146.3671) (end 215.9311 147.3713) (width 0.254) (layer F.Cu) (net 1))
 (segment (start 212.4967 146.3671) (end 214.9269 146.3671) (width 0.254) (layer F.Cu) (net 1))
 (segment (start 211.0135 144.8839) (end 212.4967 146.3671) (width 0.254) (layer F.Cu) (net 1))
 (segment (start 207.9562 144.8839) (end 211.0135 144.8839) (width 0.254) (layer F.Cu) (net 1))
 (segment (start 206.8191 146.021) (end 207.9562 144.8839) (width 0.254) (layer F.Cu) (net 1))
 (segment (start 206.8191 147.4664) (end 206.8191 146.021) (width 0.254) (layer F.Cu) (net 1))
 (segment (start 205.9845 148.301) (end 206.8191 147.4664) (width 0.254) (layer F.Cu) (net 1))
 (segment (start 202.103 148.301) (end 205.9845 148.301) (width 0.254) (layer F.Cu) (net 1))
 (segment (start 195.076 155.328) (end 202.103 148.301) (width 0.254) (layer F.Cu) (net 1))
 (segment (start 222.2177 144.2941) (end 223.7638 142.748) (width 0.254) (layer F.Cu) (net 1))
 (segment (start 220.0092 144.2941) (end 222.2177 144.2941) (width 0.254) (layer F.Cu) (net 1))
 (segment (start 216.932 147.3713) (end 220.0092 144.2941) (width 0.254) (layer F.Cu) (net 1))
 (via (at 225.1012 158.521) (size 0.889) (layers F.Cu B.Cu) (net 2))
 (via (at 208.9504 145.7239) (size 0.889) (layers F.Cu B.Cu) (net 2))
 (via (at 221.1061 143.0712) (size 0.889) (layers F.Cu B.Cu) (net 2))
 (segment (start 225.4501 158.1721) (end 225.4501 158.1404) (width 0.254) (layer F.Cu) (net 2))
 (segment (start 225.1012 158.521) (end 225.4501 158.1721) (width 0.254) (layer F.Cu) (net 2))
 (segment (start 227.2284 158.1404) (end 225.4501 158.1404) (width 0.254) (layer F.Cu) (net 2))
 (segment (start 209.1426 145.7239) (end 209.2807 145.862) (width 0.254) (layer F.Cu) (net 2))
 (segment (start 208.9504 145.7239) (end 209.1426 145.7239) (width 0.254) (layer F.Cu) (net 2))
 (segment (start 210.312 145.862) (end 209.2807 145.862) (width 0.254) (layer F.Cu) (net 2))
 (segment (start 222.2602 142.748) (end 221.4293 142.748) (width 0.254) (layer F.Cu) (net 2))
 (segment (start 221.4293 142.748) (end 221.1061 143.0712) (width 0.254) (layer F.Cu) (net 2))
 (segment (start 223.5197 146.812) (end 225.4501 148.7424) (width 0.254) (layer F.Cu) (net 4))
 (segment (start 218.932 146.812) (end 223.5197 146.812) (width 0.254) (layer F.Cu) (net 4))
 (segment (start 227.2284 148.7424) (end 225.4501 148.7424) (width 0.254) (layer F.Cu) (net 4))
 (segment (start 207.772 155.048) (end 207.772 155.448) (width 0.254) (layer B.Cu) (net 6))
 (segment (start 218.8407 143.9793) (end 207.772 155.048) (width 0.254) (layer B.Cu) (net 6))
 (segment (start 228.6312 143.9793) (end 218.8407 143.9793) (width 0.254) (layer B.Cu) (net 6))
 (segment (start 229.4007 143.2098) (end 228.6312 143.9793) (width 0.254) (layer B.Cu) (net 6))
 (segment (start 229.4007 142.748) (end 229.4007 143.2098) (width 0.254) (layer B.Cu) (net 6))
 (segment (start 230.632 142.748) (end 229.4007 142.748) (width 0.254) (layer B.Cu) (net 6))
 (segment (start 207.518 146.812) (end 207.518 147.7648) (width 0.254) (layer F.Cu) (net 6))
 (segment (start 208.0188 155.2012) (end 207.772 155.448) (width 0.254) (layer F.Cu) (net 6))
 (segment (start 208.0188 148.2656) (end 208.0188 155.2012) (width 0.254) (layer F.Cu) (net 6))
 (segment (start 207.518 147.7648) (end 208.0188 148.2656) (width 0.254) (layer F.Cu) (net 6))
 (segment (start 215.1408 145.862) (end 214.8208 145.542) (width 0.254) (layer F.Cu) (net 8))
 (segment (start 216.932 145.862) (end 215.1408 145.862) (width 0.254) (layer F.Cu) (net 8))
 (segment (start 213.868 145.542) (end 214.8208 145.542) (width 0.254) (layer F.Cu) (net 8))
 (segment (start 210.272 155.448) (end 212.772 155.448) (width 0.254) (layer F.Cu) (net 9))
 (segment (start 210.272 148.5333) (end 210.272 155.448) (width 0.254) (layer F.Cu) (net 9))
 (segment (start 210.312 148.4933) (end 210.272 148.5333) (width 0.254) (layer F.Cu) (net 9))
 (segment (start 210.312 147.762) (end 210.312 148.4933) (width 0.254) (layer F.Cu) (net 9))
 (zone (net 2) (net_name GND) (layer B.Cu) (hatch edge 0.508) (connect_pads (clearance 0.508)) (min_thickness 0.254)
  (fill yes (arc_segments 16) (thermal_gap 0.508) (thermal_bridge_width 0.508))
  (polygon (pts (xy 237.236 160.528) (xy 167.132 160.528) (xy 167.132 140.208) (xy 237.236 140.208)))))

